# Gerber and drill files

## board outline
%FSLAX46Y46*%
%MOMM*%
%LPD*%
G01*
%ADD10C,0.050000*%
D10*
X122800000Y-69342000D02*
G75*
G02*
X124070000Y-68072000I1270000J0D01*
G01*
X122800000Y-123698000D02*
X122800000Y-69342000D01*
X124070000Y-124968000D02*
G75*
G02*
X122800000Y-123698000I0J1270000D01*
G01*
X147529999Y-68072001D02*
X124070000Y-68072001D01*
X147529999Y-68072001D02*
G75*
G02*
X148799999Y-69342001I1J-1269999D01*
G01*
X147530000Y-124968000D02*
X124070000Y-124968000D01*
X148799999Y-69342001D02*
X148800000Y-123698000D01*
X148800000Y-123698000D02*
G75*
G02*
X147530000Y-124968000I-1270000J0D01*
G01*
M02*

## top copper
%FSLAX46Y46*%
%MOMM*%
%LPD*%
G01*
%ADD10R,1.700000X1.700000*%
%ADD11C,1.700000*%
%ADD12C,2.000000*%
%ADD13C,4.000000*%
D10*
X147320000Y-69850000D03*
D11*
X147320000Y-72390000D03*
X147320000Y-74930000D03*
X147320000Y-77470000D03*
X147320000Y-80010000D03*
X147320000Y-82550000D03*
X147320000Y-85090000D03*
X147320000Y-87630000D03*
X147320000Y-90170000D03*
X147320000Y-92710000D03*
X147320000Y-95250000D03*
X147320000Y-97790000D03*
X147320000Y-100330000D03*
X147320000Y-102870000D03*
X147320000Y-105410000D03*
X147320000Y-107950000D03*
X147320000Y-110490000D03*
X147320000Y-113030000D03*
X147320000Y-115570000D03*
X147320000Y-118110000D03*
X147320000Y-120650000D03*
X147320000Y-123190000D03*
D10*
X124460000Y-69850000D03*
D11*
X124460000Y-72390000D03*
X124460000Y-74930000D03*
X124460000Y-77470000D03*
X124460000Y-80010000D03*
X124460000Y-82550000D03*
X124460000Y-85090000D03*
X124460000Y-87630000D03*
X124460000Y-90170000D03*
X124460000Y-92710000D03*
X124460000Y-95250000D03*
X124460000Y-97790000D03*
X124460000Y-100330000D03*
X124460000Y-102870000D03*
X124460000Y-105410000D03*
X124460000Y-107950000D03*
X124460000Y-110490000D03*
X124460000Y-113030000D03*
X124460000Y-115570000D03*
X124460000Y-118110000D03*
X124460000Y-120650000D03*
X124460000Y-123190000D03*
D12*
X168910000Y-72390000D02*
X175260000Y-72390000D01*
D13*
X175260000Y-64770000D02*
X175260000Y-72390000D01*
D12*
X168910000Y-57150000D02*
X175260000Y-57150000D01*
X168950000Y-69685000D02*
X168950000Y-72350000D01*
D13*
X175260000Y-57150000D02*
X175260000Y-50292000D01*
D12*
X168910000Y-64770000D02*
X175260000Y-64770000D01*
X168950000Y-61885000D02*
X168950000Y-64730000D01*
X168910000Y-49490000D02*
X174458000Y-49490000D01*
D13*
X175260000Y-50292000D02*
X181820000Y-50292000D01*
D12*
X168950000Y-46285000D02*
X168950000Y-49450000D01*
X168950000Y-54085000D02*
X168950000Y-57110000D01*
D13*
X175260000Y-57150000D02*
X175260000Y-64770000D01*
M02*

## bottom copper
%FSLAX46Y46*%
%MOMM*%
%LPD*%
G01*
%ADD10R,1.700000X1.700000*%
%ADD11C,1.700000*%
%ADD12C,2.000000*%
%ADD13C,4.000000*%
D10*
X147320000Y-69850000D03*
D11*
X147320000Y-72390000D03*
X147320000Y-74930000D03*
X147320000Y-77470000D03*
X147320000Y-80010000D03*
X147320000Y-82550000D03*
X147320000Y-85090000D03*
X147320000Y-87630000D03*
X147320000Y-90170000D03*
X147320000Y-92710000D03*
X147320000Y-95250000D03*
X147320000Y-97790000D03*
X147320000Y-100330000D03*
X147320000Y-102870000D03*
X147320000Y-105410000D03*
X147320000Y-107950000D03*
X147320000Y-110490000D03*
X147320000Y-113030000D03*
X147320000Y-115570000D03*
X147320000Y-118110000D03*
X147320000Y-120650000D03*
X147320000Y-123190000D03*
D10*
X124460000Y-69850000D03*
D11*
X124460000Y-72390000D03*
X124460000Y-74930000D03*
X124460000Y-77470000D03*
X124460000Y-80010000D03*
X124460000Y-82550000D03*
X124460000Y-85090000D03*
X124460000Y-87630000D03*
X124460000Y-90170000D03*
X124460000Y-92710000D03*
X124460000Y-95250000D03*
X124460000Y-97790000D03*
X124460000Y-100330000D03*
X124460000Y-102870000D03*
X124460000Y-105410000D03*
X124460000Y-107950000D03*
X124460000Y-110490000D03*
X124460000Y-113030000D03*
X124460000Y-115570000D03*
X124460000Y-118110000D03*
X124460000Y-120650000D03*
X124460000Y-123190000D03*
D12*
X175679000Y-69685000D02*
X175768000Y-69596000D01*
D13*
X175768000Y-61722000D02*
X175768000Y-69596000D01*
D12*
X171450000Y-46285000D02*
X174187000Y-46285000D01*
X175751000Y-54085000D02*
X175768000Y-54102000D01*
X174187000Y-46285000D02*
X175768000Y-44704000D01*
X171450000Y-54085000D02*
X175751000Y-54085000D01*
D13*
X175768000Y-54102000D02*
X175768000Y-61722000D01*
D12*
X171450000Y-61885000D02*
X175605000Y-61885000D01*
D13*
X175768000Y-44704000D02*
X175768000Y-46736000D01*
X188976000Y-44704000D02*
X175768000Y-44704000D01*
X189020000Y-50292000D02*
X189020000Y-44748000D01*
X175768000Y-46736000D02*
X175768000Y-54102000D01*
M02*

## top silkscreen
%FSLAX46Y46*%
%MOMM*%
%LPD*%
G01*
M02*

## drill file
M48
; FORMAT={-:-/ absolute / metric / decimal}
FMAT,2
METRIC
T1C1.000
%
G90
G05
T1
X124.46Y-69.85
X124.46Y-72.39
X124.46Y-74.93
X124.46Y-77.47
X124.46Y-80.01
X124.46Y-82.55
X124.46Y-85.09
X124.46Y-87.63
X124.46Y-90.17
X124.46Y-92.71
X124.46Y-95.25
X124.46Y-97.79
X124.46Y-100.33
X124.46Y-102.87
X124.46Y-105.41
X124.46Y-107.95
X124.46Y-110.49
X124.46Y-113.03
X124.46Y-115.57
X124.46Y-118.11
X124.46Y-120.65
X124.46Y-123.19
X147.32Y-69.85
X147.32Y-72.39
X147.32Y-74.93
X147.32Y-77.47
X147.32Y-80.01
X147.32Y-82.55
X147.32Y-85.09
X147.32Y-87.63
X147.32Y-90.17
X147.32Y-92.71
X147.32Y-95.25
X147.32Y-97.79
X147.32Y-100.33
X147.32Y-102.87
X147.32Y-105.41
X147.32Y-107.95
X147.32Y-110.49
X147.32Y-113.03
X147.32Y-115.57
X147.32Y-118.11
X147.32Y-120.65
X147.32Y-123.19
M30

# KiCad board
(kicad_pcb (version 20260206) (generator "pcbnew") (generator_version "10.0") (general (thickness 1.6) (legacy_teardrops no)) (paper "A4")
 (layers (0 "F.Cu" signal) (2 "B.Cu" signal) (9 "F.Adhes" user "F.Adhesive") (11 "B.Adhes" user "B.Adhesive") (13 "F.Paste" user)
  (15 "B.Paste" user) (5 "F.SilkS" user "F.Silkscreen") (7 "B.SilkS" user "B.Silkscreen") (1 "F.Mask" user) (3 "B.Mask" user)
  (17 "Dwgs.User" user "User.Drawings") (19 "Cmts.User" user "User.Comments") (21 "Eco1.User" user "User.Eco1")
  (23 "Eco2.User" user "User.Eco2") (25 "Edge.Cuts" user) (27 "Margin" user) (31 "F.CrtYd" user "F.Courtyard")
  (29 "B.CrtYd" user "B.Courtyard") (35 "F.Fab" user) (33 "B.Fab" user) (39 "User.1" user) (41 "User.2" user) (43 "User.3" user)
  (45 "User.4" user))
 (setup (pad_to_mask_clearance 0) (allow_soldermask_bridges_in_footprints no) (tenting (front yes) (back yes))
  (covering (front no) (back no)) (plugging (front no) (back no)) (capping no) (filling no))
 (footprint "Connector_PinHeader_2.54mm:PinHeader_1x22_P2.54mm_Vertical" (layer "B.Cu") (at 147.32 69.85 180)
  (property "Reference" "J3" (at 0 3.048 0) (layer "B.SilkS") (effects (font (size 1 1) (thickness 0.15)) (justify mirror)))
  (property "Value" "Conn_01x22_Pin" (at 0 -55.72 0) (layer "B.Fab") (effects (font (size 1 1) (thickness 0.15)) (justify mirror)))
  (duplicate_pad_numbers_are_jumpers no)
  (pad "1" thru_hole rect (at 0 0 180) (size 1.7 1.7) (drill 1) (layers "*.Cu" "*.Mask") (remove_unused_layers no) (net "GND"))
  (pad "2" thru_hole circle (at 0 -2.54 180) (size 1.7 1.7) (drill 1) (layers "*.Cu" "*.Mask") (remove_unused_layers no) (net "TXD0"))
  (pad "3" thru_hole circle (at 0 -5.08 180) (size 1.7 1.7) (drill 1) (layers "*.Cu" "*.Mask") (remove_unused_layers no) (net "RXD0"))
  (pad "4" thru_hole circle (at 0 -7.62 180) (size 1.7 1.7) (drill 1) (layers "*.Cu" "*.Mask") (remove_unused_layers no) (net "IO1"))
  (pad "5" thru_hole circle (at 0 -10.16 180) (size 1.7 1.7) (drill 1) (layers "*.Cu" "*.Mask") (remove_unused_layers no) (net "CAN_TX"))
  (pad "6" thru_hole circle (at 0 -12.7 180) (size 1.7 1.7) (drill 1) (layers "*.Cu" "*.Mask") (remove_unused_layers no) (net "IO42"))
  (pad "7" thru_hole circle (at 0 -15.24 180) (size 1.7 1.7) (drill 1) (layers "*.Cu" "*.Mask") (remove_unused_layers no) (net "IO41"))
  (pad "8" thru_hole circle (at 0 -17.78 180) (size 1.7 1.7) (drill 1) (layers "*.Cu" "*.Mask") (remove_unused_layers no) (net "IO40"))
  (pad "9" thru_hole circle (at 0 -20.32 180) (size 1.7 1.7) (drill 1) (layers "*.Cu" "*.Mask") (remove_unused_layers no) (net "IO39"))
  (pad "10" thru_hole circle (at 0 -22.86 180) (size 1.7 1.7) (drill 1) (layers "*.Cu" "*.Mask") (remove_unused_layers no) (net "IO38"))
  (pad "11" thru_hole circle (at 0 -25.4 180) (size 1.7 1.7) (drill 1) (layers "*.Cu" "*.Mask") (remove_unused_layers no) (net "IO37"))
  (pad "12" thru_hole circle (at 0 -27.94 180) (size 1.7 1.7) (drill 1) (layers "*.Cu" "*.Mask") (remove_unused_layers no) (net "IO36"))
  (pad "13" thru_hole circle (at 0 -30.48 180) (size 1.7 1.7) (drill 1) (layers "*.Cu" "*.Mask") (remove_unused_layers no) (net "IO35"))
  (pad "14" thru_hole circle (at 0 -33.02 180) (size 1.7 1.7) (drill 1) (layers "*.Cu" "*.Mask") (remove_unused_layers no) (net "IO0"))
  (pad "15" thru_hole circle (at 0 -35.56 180) (size 1.7 1.7) (drill 1) (layers "*.Cu" "*.Mask") (remove_unused_layers no) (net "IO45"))
  (pad "16" thru_hole circle (at 0 -38.1 180) (size 1.7 1.7) (drill 1) (layers "*.Cu" "*.Mask") (remove_unused_layers no) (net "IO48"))
  (pad "17" thru_hole circle (at 0 -40.64 180) (size 1.7 1.7) (drill 1) (layers "*.Cu" "*.Mask") (remove_unused_layers no) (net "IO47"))
  (pad "18" thru_hole circle (at 0 -43.18 180) (size 1.7 1.7) (drill 1) (layers "*.Cu" "*.Mask") (remove_unused_layers no) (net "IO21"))
  (pad "19" thru_hole circle (at 0 -45.72 180) (size 1.7 1.7) (drill 1) (layers "*.Cu" "*.Mask") (remove_unused_layers no) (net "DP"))
  (pad "20" thru_hole circle (at 0 -48.26 180) (size 1.7 1.7) (drill 1) (layers "*.Cu" "*.Mask") (remove_unused_layers no) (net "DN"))
  (pad "21" thru_hole circle (at 0 -50.8 180) (size 1.7 1.7) (drill 1) (layers "*.Cu" "*.Mask") (remove_unused_layers no) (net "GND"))
  (pad "22" thru_hole circle (at 0 -53.34 180) (size 1.7 1.7) (drill 1) (layers "*.Cu" "*.Mask") (remove_unused_layers no) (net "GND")))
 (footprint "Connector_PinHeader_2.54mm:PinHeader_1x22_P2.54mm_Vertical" (layer "B.Cu") (at 124.46 69.85 180)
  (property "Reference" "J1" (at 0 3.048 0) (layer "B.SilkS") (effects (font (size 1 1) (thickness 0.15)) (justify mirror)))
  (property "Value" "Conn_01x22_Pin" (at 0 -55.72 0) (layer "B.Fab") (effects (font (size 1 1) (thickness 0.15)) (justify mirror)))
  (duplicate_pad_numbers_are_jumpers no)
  (pad "1" thru_hole rect (at 0 0 180) (size 1.7 1.7) (drill 1) (layers "*.Cu" "*.Mask") (remove_unused_layers no) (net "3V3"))
  (pad "2" thru_hole circle (at 0 -2.54 180) (size 1.7 1.7) (drill 1) (layers "*.Cu" "*.Mask") (remove_unused_layers no) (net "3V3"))
  (pad "3" thru_hole circle (at 0 -5.08 180) (size 1.7 1.7) (drill 1) (layers "*.Cu" "*.Mask") (remove_unused_layers no) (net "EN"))
  (pad "4" thru_hole circle (at 0 -7.62 180) (size 1.7 1.7) (drill 1) (layers "*.Cu" "*.Mask") (remove_unused_layers no) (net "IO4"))
  (pad "5" thru_hole circle (at 0 -10.16 180) (size 1.7 1.7) (drill 1) (layers "*.Cu" "*.Mask") (remove_unused_layers no) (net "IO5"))
  (pad "6" thru_hole circle (at 0 -12.7 180) (size 1.7 1.7) (drill 1) (layers "*.Cu" "*.Mask") (remove_unused_layers no) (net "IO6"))
  (pad "7" thru_hole circle (at 0 -15.24 180) (size 1.7 1.7) (drill 1) (layers "*.Cu" "*.Mask") (remove_unused_layers no) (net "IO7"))
  (pad "8" thru_hole circle (at 0 -17.78 180) (size 1.7 1.7) (drill 1) (layers "*.Cu" "*.Mask") (remove_unused_layers no) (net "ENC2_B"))
  (pad "9" thru_hole circle (at 0 -20.32 180) (size 1.7 1.7) (drill 1) (layers "*.Cu" "*.Mask") (remove_unused_layers no) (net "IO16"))
  (pad "10" thru_hole circle (at 0 -22.86 180) (size 1.7 1.7) (drill 1) (layers "*.Cu" "*.Mask") (remove_unused_layers no) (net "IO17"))
  (pad "11" thru_hole circle (at 0 -25.4 180) (size 1.7 1.7) (drill 1) (layers "*.Cu" "*.Mask") (remove_unused_layers no) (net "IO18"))
  (pad "12" thru_hole circle (at 0 -27.94 180) (size 1.7 1.7) (drill 1) (layers "*.Cu" "*.Mask") (remove_unused_layers no) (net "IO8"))
  (pad "13" thru_hole circle (at 0 -30.48 180) (size 1.7 1.7) (drill 1) (layers "*.Cu" "*.Mask") (remove_unused_layers no) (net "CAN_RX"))
  (pad "14" thru_hole circle (at 0 -33.02 180) (size 1.7 1.7) (drill 1) (layers "*.Cu" "*.Mask") (remove_unused_layers no) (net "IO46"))
  (pad "15" thru_hole circle (at 0 -35.56 180) (size 1.7 1.7) (drill 1) (layers "*.Cu" "*.Mask") (remove_unused_layers no) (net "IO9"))
  (pad "16" thru_hole circle (at 0 -38.1 180) (size 1.7 1.7) (drill 1) (layers "*.Cu" "*.Mask") (remove_unused_layers no) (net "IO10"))
  (pad "17" thru_hole circle (at 0 -40.64 180) (size 1.7 1.7) (drill 1) (layers "*.Cu" "*.Mask") (remove_unused_layers no) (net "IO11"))
  (pad "18" thru_hole circle (at 0 -43.18 180) (size 1.7 1.7) (drill 1) (layers "*.Cu" "*.Mask") (remove_unused_layers no) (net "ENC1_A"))
  (pad "19" thru_hole circle (at 0 -45.72 180) (size 1.7 1.7) (drill 1) (layers "*.Cu" "*.Mask") (remove_unused_layers no) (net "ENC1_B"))
  (pad "20" thru_hole circle (at 0 -48.26 180) (size 1.7 1.7) (drill 1) (layers "*.Cu" "*.Mask") (remove_unused_layers no) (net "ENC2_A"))
  (pad "21" thru_hole circle (at 0 -50.8 180) (size 1.7 1.7) (drill 1) (layers "*.Cu" "*.Mask") (remove_unused_layers no) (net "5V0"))
  (pad "22" thru_hole circle (at 0 -53.34 180) (size 1.7 1.7) (drill 1) (layers "*.Cu" "*.Mask") (remove_unused_layers no) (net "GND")))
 (gr_arc (start 122.8 69.342) (mid 123.171974 68.443974) (end 124.07 68.072) (stroke (width 0.05) (type default)) (layer "Edge.Cuts"))
 (gr_line (start 122.8 123.698) (end 122.8 69.342) (stroke (width 0.05) (type default)) (layer "Edge.Cuts"))
 (gr_arc (start 124.07 124.968) (mid 123.171974 124.596026) (end 122.8 123.698) (stroke (width 0.05) (type default)) (layer "Edge.Cuts"))
 (gr_line (start 147.529999 68.072001) (end 124.07 68.072001) (stroke (width 0.05) (type default)) (layer "Edge.Cuts"))
 (gr_arc (start 147.529999 68.072001) (mid 148.428025 68.443975) (end 148.799999 69.342001) (stroke (width 0.05) (type default))
  (layer "Edge.Cuts"))
 (gr_line (start 147.53 124.968) (end 124.07 124.968) (stroke (width 0.05) (type default)) (layer "Edge.Cuts"))
 (gr_line (start 148.799999 69.342001) (end 148.8 123.698) (stroke (width 0.05) (type default)) (layer "Edge.Cuts"))
 (gr_arc (start 148.8 123.698) (mid 148.428026 124.596026) (end 147.53 124.968) (stroke (width 0.05) (type default)) (layer "Edge.Cuts"))
 (segment (start 175.679 69.685) (end 175.768 69.596) (width 2) (locked yes) (layer "B.Cu") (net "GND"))
 (segment (start 175.768 61.722) (end 175.768 69.596) (width 4) (locked yes) (layer "B.Cu") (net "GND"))
 (segment (start 171.45 46.285) (end 174.187 46.285) (width 2) (locked yes) (layer "B.Cu") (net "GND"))
 (segment (start 175.751 54.085) (end 175.768 54.102) (width 2) (locked yes) (layer "B.Cu") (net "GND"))
 (segment (start 174.187 46.285) (end 175.768 44.704) (width 2) (locked yes) (layer "B.Cu") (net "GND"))
 (segment (start 171.45 54.085) (end 175.751 54.085) (width 2) (locked yes) (layer "B.Cu") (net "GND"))
 (segment (start 175.768 54.102) (end 175.768 61.722) (width 4) (locked yes) (layer "B.Cu") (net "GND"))
 (segment (start 171.45 61.885) (end 175.605 61.885) (width 2) (locked yes) (layer "B.Cu") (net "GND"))
 (segment (start 175.768 44.704) (end 175.768 46.736) (width 4) (locked yes) (layer "B.Cu") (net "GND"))
 (segment (start 188.976 44.704) (end 175.768 44.704) (width 4) (locked yes) (layer "B.Cu") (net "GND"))
 (segment (start 189.02 50.292) (end 189.02 44.748) (width 4) (locked yes) (layer "B.Cu") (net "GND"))
 (segment (start 175.768 46.736) (end 175.768 54.102) (width 4) (locked yes) (layer "B.Cu") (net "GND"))
 (segment (start 168.91 72.39) (end 175.26 72.39) (width 2) (locked yes) (layer "F.Cu") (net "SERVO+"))
 (segment (start 175.26 64.77) (end 175.26 72.39) (width 4) (locked yes) (layer "F.Cu") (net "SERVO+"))
 (segment (start 168.91 57.15) (end 175.26 57.15) (width 2) (locked yes) (layer "F.Cu") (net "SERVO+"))
 (segment (start 168.95 69.685) (end 168.95 72.35) (width 2) (locked yes) (layer "F.Cu") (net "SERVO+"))
 (segment (start 175.26 57.15) (end 175.26 50.292) (width 4) (locked yes) (layer "F.Cu") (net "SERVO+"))
 (segment (start 168.91 64.77) (end 175.26 64.77) (width 2) (locked yes) (layer "F.Cu") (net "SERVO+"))
 (segment (start 168.95 61.885) (end 168.95 64.73) (width 2) (locked yes) (layer "F.Cu") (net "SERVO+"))
 (segment (start 168.91 49.49) (end 174.458 49.49) (width 2) (locked yes) (layer "F.Cu") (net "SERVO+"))
 (segment (start 175.26 50.292) (end 181.82 50.292) (width 4) (locked yes) (layer "F.Cu") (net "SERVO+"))
 (segment (start 168.95 46.285) (end 168.95 49.45) (width 2) (locked yes) (layer "F.Cu") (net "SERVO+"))
 (segment (start 168.95 54.085) (end 168.95 57.11) (width 2) (locked yes) (layer "F.Cu") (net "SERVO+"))
 (segment (start 175.26 57.15) (end 175.26 64.77) (width 4) (locked yes) (layer "F.Cu") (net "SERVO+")))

